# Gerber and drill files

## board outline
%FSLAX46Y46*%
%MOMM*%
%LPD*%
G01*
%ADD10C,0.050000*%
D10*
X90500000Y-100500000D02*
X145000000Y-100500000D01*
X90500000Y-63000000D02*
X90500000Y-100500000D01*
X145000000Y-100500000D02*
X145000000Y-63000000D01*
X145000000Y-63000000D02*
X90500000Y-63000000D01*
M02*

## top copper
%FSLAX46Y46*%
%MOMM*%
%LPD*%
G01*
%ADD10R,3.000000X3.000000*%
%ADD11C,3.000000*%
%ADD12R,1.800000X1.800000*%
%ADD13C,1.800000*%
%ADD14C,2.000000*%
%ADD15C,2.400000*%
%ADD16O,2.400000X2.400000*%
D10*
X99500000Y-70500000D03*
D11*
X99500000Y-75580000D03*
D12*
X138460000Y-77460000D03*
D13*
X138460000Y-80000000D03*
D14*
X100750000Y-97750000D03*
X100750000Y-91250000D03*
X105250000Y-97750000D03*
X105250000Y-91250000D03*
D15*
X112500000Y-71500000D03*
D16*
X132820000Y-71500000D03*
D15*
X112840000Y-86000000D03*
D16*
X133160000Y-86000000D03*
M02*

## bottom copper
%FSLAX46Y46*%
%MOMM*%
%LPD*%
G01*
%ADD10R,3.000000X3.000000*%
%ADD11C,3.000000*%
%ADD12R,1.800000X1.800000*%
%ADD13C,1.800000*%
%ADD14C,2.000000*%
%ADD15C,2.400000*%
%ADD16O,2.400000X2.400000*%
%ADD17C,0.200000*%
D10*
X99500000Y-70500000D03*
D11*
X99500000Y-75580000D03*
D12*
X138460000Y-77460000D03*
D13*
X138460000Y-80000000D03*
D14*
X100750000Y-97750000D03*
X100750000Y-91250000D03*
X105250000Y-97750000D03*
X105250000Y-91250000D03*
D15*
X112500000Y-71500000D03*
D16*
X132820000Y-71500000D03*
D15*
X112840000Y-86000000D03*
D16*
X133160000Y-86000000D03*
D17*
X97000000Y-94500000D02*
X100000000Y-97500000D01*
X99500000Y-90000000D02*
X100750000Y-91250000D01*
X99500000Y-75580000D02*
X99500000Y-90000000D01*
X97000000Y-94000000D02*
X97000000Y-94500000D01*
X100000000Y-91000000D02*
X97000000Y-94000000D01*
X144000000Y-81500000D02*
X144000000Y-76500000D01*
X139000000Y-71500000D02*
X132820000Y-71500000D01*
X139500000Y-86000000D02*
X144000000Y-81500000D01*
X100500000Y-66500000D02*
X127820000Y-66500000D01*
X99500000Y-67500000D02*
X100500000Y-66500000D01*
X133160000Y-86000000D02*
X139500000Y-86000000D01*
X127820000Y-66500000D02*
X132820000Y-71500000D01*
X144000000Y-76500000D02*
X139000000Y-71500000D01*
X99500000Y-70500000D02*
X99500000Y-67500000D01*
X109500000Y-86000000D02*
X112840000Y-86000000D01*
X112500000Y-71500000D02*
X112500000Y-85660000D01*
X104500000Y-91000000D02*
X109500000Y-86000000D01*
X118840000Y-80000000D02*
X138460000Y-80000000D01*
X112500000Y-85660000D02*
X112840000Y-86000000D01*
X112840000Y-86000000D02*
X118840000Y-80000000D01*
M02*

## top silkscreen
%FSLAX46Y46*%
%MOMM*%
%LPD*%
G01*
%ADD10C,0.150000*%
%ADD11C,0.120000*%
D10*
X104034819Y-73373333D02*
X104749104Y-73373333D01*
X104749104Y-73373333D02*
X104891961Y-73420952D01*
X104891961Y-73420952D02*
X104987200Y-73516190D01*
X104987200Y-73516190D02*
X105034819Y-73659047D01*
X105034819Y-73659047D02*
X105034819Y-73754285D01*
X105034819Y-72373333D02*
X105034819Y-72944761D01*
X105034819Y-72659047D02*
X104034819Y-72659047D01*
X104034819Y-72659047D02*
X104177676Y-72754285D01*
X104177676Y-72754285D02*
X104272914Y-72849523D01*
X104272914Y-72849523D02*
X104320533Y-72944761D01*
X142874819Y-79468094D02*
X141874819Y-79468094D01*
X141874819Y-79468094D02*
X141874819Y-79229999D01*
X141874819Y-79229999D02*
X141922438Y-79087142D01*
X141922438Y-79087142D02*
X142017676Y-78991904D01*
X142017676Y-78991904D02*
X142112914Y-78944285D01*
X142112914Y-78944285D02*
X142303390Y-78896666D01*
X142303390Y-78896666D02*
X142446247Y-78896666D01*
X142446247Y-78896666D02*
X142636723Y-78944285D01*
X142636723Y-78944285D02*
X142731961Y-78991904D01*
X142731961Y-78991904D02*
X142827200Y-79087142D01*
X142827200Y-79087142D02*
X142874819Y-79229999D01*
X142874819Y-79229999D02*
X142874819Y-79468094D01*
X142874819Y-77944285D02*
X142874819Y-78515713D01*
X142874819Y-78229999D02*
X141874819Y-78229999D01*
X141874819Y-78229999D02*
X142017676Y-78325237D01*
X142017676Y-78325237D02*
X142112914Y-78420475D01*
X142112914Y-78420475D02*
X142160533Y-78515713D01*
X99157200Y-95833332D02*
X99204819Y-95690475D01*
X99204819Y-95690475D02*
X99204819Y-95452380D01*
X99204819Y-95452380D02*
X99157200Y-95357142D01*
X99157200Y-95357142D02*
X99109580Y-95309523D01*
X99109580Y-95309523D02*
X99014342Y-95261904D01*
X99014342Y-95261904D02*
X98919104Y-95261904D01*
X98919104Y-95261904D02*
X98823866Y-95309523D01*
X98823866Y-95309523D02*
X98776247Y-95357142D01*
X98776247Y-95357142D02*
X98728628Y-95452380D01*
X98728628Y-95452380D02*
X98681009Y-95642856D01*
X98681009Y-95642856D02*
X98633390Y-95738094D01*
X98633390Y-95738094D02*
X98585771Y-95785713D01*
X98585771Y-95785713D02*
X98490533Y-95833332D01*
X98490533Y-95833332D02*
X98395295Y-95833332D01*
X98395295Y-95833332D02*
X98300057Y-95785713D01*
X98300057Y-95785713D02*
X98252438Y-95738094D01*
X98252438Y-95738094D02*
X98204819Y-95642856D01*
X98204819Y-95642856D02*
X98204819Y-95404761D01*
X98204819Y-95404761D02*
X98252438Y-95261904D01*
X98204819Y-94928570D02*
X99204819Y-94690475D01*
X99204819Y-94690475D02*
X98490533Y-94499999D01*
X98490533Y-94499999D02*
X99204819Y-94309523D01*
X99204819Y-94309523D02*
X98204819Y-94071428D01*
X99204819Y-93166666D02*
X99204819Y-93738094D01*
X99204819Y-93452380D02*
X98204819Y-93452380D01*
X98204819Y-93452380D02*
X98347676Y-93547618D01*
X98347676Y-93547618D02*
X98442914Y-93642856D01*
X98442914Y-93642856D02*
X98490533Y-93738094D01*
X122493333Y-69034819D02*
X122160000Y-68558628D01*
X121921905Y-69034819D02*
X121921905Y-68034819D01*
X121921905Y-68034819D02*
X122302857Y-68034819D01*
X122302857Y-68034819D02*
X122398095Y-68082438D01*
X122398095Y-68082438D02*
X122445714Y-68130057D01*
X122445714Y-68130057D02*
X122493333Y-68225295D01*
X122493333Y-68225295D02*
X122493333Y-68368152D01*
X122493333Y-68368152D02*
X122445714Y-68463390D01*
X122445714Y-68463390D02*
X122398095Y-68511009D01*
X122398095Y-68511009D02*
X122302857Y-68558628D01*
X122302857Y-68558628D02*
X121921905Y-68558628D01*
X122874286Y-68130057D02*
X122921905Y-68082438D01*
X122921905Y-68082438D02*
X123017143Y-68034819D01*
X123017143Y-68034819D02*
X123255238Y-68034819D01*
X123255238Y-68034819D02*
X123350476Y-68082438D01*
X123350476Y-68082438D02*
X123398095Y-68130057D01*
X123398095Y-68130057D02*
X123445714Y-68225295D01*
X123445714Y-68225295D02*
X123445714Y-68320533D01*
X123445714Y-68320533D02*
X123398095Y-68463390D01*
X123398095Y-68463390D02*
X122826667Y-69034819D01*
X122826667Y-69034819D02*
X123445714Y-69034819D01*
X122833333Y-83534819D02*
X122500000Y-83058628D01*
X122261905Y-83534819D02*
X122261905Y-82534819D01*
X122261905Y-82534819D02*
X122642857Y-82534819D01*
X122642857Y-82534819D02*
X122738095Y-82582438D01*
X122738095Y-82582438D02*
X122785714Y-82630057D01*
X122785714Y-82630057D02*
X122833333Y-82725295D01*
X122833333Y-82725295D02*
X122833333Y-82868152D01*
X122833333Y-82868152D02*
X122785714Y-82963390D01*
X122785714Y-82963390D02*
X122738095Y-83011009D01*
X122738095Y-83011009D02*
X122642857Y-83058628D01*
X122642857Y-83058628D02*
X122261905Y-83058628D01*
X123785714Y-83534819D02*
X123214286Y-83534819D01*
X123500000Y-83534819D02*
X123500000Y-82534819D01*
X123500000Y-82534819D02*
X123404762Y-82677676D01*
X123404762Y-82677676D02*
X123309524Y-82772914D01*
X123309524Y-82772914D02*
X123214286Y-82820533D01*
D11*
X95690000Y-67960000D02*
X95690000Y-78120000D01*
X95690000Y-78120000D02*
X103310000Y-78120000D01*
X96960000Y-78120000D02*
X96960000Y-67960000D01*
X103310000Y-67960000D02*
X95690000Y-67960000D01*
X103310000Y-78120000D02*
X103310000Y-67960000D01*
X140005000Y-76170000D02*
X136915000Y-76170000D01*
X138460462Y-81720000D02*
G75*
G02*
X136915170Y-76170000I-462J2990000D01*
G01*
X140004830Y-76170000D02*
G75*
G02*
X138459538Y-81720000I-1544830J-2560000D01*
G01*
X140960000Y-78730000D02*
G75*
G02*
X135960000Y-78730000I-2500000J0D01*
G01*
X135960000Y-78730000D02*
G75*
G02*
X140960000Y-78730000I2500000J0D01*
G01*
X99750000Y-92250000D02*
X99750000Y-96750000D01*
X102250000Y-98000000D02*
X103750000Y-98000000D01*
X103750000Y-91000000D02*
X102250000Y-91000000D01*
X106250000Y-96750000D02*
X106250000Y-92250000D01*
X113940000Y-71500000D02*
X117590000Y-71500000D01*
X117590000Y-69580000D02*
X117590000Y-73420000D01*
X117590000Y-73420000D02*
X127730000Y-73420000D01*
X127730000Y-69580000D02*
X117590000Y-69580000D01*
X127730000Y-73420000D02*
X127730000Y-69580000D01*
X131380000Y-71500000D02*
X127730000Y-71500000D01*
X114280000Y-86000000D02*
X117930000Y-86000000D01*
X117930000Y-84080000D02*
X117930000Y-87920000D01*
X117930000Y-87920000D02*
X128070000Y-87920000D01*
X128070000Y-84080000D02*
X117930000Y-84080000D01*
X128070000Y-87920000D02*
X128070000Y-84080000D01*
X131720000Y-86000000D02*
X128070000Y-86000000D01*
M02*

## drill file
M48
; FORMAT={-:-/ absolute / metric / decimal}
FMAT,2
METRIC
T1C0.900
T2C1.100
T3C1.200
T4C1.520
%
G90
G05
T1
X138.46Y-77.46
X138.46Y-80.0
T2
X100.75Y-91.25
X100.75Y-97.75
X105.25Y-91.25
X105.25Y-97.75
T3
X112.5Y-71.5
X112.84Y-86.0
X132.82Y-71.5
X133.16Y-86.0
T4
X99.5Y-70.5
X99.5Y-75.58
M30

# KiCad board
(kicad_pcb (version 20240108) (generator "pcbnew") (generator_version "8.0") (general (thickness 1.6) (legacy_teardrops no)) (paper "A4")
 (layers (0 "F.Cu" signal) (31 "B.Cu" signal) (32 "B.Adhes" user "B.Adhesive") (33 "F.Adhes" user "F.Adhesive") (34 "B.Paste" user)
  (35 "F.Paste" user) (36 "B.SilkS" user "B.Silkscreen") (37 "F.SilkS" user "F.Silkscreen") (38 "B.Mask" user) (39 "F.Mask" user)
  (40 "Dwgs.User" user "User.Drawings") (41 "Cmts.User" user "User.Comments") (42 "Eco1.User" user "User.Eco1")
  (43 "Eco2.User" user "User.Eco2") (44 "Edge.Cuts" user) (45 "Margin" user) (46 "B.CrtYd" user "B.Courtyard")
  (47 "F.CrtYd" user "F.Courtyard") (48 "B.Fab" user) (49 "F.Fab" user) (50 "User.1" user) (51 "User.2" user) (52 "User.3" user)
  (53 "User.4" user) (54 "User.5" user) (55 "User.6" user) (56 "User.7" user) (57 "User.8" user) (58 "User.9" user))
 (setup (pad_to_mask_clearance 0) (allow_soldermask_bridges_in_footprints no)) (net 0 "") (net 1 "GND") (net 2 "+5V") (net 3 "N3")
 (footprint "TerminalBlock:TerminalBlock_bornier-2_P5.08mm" (layer "F.Cu") (at 99.5 70.5 -90)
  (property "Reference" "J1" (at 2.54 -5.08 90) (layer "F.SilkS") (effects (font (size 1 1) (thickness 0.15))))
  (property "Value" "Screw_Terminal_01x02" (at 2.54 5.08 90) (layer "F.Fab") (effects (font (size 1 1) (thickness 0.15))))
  (fp_line (start -2.54 3.81) (end 7.62 3.81) (stroke (width 0.12) (type solid)) (layer "F.SilkS"))
  (fp_line (start 7.62 3.81) (end 7.62 -3.81) (stroke (width 0.12) (type solid)) (layer "F.SilkS"))
  (fp_line (start 7.62 2.54) (end -2.54 2.54) (stroke (width 0.12) (type solid)) (layer "F.SilkS"))
  (fp_line (start -2.54 -3.81) (end -2.54 3.81) (stroke (width 0.12) (type solid)) (layer "F.SilkS"))
  (fp_line (start 7.62 -3.81) (end -2.54 -3.81) (stroke (width 0.12) (type solid)) (layer "F.SilkS"))
  (pad "1" thru_hole rect (at 0 0 270) (size 3 3) (drill 1.52) (layers "*.Cu" "*.Mask") (remove_unused_layers no) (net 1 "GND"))
  (pad "2" thru_hole circle (at 5.08 0 270) (size 3 3) (drill 1.52) (layers "*.Cu" "*.Mask") (remove_unused_layers no) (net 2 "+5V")))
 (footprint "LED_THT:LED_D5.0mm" (layer "F.Cu") (at 138.46 77.46 -90)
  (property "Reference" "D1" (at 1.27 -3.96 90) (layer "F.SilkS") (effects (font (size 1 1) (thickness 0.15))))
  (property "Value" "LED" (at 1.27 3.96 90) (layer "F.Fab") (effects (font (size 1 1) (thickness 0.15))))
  (fp_line (start -1.29 -1.545) (end -1.29 1.545) (stroke (width 0.12) (type solid)) (layer "F.SilkS"))
  (fp_arc (start 4.26 -0.000462) (mid 2.072002 2.880433) (end -1.29 1.54483) (stroke (width 0.12) (type solid)) (layer "F.SilkS"))
  (fp_arc (start -1.29 -1.54483) (mid 2.072002 -2.880433) (end 4.26 0.000462) (stroke (width 0.12) (type solid)) (layer "F.SilkS"))
  (fp_circle (center 1.27 0) (end 3.77 0) (stroke (width 0.12) (type solid)) (fill none) (layer "F.SilkS"))
  (pad "1" thru_hole rect (at 0 0 270) (size 1.8 1.8) (drill 0.9) (layers "*.Cu" "*.Mask") (remove_unused_layers no) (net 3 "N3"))
  (pad "2" thru_hole circle (at 2.54 0 270) (size 1.8 1.8) (drill 0.9) (layers "*.Cu" "*.Mask") (remove_unused_layers no) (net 3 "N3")))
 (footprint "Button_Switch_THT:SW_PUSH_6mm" (layer "F.Cu") (at 100.75 97.75 90)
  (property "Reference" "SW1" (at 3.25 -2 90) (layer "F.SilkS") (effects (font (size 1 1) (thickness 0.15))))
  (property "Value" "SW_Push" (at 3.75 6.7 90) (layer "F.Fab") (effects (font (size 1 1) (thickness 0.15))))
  (fp_line (start 5.5 -1) (end 1 -1) (stroke (width 0.12) (type solid)) (layer "F.SilkS"))
  (fp_line (start -0.25 1.5) (end -0.25 3) (stroke (width 0.12) (type solid)) (layer "F.SilkS"))
  (fp_line (start 6.75 3) (end 6.75 1.5) (stroke (width 0.12) (type solid)) (layer "F.SilkS"))
  (fp_line (start 1 5.5) (end 5.5 5.5) (stroke (width 0.12) (type solid)) (layer "F.SilkS"))
  (pad "1" thru_hole circle (at 0 0 180) (size 2 2) (drill 1.1) (layers "*.Cu" "*.Mask") (remove_unused_layers no) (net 2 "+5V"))
  (pad "1" thru_hole circle (at 6.5 0 180) (size 2 2) (drill 1.1) (layers "*.Cu" "*.Mask") (remove_unused_layers no) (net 2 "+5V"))
  (pad "2" thru_hole circle (at 0 4.5 180) (size 2 2) (drill 1.1) (layers "*.Cu" "*.Mask") (remove_unused_layers no) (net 3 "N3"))
  (pad "2" thru_hole circle (at 6.5 4.5 180) (size 2 2) (drill 1.1) (layers "*.Cu" "*.Mask") (remove_unused_layers no) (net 3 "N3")))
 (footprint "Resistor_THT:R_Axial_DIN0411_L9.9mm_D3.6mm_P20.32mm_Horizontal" (layer "F.Cu") (at 112.5 71.5)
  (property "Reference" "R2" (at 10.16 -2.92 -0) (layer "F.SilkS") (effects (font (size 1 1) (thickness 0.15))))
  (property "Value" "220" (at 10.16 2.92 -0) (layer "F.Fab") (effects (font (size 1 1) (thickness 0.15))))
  (fp_line (start 1.44 0) (end 5.09 0) (stroke (width 0.12) (type solid)) (layer "F.SilkS"))
  (fp_line (start 5.09 -1.92) (end 5.09 1.92) (stroke (width 0.12) (type solid)) (layer "F.SilkS"))
  (fp_line (start 5.09 1.92) (end 15.23 1.92) (stroke (width 0.12) (type solid)) (layer "F.SilkS"))
  (fp_line (start 15.23 -1.92) (end 5.09 -1.92) (stroke (width 0.12) (type solid)) (layer "F.SilkS"))
  (fp_line (start 15.23 1.92) (end 15.23 -1.92) (stroke (width 0.12) (type solid)) (layer "F.SilkS"))
  (fp_line (start 18.88 0) (end 15.23 0) (stroke (width 0.12) (type solid)) (layer "F.SilkS"))
  (pad "1" thru_hole circle (at 0 0) (size 2.4 2.4) (drill 1.2) (layers "*.Cu" "*.Mask") (remove_unused_layers no) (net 3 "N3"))
  (pad "2" thru_hole oval (at 20.32 0) (size 2.4 2.4) (drill 1.2) (layers "*.Cu" "*.Mask") (remove_unused_layers no) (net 1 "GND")))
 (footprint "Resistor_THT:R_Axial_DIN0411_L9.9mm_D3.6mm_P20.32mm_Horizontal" (layer "F.Cu") (at 112.84 86)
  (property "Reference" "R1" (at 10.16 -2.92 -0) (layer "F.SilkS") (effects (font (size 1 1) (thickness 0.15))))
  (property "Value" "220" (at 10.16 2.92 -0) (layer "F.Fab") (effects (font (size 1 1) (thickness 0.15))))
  (fp_line (start 1.44 0) (end 5.09 0) (stroke (width 0.12) (type solid)) (layer "F.SilkS"))
  (fp_line (start 5.09 -1.92) (end 5.09 1.92) (stroke (width 0.12) (type solid)) (layer "F.SilkS"))
  (fp_line (start 5.09 1.92) (end 15.23 1.92) (stroke (width 0.12) (type solid)) (layer "F.SilkS"))
  (fp_line (start 15.23 -1.92) (end 5.09 -1.92) (stroke (width 0.12) (type solid)) (layer "F.SilkS"))
  (fp_line (start 15.23 1.92) (end 15.23 -1.92) (stroke (width 0.12) (type solid)) (layer "F.SilkS"))
  (fp_line (start 18.88 0) (end 15.23 0) (stroke (width 0.12) (type solid)) (layer "F.SilkS"))
  (pad "1" thru_hole circle (at 0 0) (size 2.4 2.4) (drill 1.2) (layers "*.Cu" "*.Mask") (remove_unused_layers no) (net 3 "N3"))
  (pad "2" thru_hole oval (at 20.32 0) (size 2.4 2.4) (drill 1.2) (layers "*.Cu" "*.Mask") (remove_unused_layers no) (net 1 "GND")))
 (gr_line (start 90.5 100.5) (end 145 100.5) (stroke (width 0.05) (type default)) (layer "Edge.Cuts"))
 (gr_line (start 90.5 63) (end 90.5 100.5) (stroke (width 0.05) (type default)) (layer "Edge.Cuts"))
 (gr_line (start 145 100.5) (end 145 63) (stroke (width 0.05) (type default)) (layer "Edge.Cuts"))
 (gr_line (start 145 63) (end 90.5 63) (stroke (width 0.05) (type default)) (layer "Edge.Cuts"))
 (segment (start 97 94.5) (end 100 97.5) (width 0.2) (layer "B.Cu") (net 2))
 (segment (start 99.5 90) (end 100.75 91.25) (width 0.2) (layer "B.Cu") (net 2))
 (segment (start 99.5 75.58) (end 99.5 90) (width 0.2) (layer "B.Cu") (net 2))
 (segment (start 97 94) (end 97 94.5) (width 0.2) (layer "B.Cu") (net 2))
 (segment (start 100 91) (end 97 94) (width 0.2) (layer "B.Cu") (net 2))
 (segment (start 144 81.5) (end 144 76.5) (width 0.2) (layer "B.Cu") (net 1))
 (segment (start 139 71.5) (end 132.82 71.5) (width 0.2) (layer "B.Cu") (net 1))
 (segment (start 139.5 86) (end 144 81.5) (width 0.2) (layer "B.Cu") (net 1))
 (segment (start 100.5 66.5) (end 127.82 66.5) (width 0.2) (layer "B.Cu") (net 1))
 (segment (start 99.5 67.5) (end 100.5 66.5) (width 0.2) (layer "B.Cu") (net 1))
 (segment (start 133.16 86) (end 139.5 86) (width 0.2) (layer "B.Cu") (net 1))
 (segment (start 127.82 66.5) (end 132.82 71.5) (width 0.2) (layer "B.Cu") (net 1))
 (segment (start 144 76.5) (end 139 71.5) (width 0.2) (layer "B.Cu") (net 1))
 (segment (start 99.5 70.5) (end 99.5 67.5) (width 0.2) (layer "B.Cu") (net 1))
 (segment (start 109.5 86) (end 112.84 86) (width 0.2) (layer "B.Cu") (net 3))
 (segment (start 112.5 71.5) (end 112.5 85.66) (width 0.2) (layer "B.Cu") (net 3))
 (segment (start 104.5 91) (end 109.5 86) (width 0.2) (layer "B.Cu") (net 3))
 (segment (start 118.84 80) (end 138.46 80) (width 0.2) (layer "B.Cu") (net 3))
 (segment (start 112.5 85.66) (end 112.84 86) (width 0.2) (layer "B.Cu") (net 3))
 (segment (start 112.84 86) (end 118.84 80) (width 0.2) (layer "B.Cu") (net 3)))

